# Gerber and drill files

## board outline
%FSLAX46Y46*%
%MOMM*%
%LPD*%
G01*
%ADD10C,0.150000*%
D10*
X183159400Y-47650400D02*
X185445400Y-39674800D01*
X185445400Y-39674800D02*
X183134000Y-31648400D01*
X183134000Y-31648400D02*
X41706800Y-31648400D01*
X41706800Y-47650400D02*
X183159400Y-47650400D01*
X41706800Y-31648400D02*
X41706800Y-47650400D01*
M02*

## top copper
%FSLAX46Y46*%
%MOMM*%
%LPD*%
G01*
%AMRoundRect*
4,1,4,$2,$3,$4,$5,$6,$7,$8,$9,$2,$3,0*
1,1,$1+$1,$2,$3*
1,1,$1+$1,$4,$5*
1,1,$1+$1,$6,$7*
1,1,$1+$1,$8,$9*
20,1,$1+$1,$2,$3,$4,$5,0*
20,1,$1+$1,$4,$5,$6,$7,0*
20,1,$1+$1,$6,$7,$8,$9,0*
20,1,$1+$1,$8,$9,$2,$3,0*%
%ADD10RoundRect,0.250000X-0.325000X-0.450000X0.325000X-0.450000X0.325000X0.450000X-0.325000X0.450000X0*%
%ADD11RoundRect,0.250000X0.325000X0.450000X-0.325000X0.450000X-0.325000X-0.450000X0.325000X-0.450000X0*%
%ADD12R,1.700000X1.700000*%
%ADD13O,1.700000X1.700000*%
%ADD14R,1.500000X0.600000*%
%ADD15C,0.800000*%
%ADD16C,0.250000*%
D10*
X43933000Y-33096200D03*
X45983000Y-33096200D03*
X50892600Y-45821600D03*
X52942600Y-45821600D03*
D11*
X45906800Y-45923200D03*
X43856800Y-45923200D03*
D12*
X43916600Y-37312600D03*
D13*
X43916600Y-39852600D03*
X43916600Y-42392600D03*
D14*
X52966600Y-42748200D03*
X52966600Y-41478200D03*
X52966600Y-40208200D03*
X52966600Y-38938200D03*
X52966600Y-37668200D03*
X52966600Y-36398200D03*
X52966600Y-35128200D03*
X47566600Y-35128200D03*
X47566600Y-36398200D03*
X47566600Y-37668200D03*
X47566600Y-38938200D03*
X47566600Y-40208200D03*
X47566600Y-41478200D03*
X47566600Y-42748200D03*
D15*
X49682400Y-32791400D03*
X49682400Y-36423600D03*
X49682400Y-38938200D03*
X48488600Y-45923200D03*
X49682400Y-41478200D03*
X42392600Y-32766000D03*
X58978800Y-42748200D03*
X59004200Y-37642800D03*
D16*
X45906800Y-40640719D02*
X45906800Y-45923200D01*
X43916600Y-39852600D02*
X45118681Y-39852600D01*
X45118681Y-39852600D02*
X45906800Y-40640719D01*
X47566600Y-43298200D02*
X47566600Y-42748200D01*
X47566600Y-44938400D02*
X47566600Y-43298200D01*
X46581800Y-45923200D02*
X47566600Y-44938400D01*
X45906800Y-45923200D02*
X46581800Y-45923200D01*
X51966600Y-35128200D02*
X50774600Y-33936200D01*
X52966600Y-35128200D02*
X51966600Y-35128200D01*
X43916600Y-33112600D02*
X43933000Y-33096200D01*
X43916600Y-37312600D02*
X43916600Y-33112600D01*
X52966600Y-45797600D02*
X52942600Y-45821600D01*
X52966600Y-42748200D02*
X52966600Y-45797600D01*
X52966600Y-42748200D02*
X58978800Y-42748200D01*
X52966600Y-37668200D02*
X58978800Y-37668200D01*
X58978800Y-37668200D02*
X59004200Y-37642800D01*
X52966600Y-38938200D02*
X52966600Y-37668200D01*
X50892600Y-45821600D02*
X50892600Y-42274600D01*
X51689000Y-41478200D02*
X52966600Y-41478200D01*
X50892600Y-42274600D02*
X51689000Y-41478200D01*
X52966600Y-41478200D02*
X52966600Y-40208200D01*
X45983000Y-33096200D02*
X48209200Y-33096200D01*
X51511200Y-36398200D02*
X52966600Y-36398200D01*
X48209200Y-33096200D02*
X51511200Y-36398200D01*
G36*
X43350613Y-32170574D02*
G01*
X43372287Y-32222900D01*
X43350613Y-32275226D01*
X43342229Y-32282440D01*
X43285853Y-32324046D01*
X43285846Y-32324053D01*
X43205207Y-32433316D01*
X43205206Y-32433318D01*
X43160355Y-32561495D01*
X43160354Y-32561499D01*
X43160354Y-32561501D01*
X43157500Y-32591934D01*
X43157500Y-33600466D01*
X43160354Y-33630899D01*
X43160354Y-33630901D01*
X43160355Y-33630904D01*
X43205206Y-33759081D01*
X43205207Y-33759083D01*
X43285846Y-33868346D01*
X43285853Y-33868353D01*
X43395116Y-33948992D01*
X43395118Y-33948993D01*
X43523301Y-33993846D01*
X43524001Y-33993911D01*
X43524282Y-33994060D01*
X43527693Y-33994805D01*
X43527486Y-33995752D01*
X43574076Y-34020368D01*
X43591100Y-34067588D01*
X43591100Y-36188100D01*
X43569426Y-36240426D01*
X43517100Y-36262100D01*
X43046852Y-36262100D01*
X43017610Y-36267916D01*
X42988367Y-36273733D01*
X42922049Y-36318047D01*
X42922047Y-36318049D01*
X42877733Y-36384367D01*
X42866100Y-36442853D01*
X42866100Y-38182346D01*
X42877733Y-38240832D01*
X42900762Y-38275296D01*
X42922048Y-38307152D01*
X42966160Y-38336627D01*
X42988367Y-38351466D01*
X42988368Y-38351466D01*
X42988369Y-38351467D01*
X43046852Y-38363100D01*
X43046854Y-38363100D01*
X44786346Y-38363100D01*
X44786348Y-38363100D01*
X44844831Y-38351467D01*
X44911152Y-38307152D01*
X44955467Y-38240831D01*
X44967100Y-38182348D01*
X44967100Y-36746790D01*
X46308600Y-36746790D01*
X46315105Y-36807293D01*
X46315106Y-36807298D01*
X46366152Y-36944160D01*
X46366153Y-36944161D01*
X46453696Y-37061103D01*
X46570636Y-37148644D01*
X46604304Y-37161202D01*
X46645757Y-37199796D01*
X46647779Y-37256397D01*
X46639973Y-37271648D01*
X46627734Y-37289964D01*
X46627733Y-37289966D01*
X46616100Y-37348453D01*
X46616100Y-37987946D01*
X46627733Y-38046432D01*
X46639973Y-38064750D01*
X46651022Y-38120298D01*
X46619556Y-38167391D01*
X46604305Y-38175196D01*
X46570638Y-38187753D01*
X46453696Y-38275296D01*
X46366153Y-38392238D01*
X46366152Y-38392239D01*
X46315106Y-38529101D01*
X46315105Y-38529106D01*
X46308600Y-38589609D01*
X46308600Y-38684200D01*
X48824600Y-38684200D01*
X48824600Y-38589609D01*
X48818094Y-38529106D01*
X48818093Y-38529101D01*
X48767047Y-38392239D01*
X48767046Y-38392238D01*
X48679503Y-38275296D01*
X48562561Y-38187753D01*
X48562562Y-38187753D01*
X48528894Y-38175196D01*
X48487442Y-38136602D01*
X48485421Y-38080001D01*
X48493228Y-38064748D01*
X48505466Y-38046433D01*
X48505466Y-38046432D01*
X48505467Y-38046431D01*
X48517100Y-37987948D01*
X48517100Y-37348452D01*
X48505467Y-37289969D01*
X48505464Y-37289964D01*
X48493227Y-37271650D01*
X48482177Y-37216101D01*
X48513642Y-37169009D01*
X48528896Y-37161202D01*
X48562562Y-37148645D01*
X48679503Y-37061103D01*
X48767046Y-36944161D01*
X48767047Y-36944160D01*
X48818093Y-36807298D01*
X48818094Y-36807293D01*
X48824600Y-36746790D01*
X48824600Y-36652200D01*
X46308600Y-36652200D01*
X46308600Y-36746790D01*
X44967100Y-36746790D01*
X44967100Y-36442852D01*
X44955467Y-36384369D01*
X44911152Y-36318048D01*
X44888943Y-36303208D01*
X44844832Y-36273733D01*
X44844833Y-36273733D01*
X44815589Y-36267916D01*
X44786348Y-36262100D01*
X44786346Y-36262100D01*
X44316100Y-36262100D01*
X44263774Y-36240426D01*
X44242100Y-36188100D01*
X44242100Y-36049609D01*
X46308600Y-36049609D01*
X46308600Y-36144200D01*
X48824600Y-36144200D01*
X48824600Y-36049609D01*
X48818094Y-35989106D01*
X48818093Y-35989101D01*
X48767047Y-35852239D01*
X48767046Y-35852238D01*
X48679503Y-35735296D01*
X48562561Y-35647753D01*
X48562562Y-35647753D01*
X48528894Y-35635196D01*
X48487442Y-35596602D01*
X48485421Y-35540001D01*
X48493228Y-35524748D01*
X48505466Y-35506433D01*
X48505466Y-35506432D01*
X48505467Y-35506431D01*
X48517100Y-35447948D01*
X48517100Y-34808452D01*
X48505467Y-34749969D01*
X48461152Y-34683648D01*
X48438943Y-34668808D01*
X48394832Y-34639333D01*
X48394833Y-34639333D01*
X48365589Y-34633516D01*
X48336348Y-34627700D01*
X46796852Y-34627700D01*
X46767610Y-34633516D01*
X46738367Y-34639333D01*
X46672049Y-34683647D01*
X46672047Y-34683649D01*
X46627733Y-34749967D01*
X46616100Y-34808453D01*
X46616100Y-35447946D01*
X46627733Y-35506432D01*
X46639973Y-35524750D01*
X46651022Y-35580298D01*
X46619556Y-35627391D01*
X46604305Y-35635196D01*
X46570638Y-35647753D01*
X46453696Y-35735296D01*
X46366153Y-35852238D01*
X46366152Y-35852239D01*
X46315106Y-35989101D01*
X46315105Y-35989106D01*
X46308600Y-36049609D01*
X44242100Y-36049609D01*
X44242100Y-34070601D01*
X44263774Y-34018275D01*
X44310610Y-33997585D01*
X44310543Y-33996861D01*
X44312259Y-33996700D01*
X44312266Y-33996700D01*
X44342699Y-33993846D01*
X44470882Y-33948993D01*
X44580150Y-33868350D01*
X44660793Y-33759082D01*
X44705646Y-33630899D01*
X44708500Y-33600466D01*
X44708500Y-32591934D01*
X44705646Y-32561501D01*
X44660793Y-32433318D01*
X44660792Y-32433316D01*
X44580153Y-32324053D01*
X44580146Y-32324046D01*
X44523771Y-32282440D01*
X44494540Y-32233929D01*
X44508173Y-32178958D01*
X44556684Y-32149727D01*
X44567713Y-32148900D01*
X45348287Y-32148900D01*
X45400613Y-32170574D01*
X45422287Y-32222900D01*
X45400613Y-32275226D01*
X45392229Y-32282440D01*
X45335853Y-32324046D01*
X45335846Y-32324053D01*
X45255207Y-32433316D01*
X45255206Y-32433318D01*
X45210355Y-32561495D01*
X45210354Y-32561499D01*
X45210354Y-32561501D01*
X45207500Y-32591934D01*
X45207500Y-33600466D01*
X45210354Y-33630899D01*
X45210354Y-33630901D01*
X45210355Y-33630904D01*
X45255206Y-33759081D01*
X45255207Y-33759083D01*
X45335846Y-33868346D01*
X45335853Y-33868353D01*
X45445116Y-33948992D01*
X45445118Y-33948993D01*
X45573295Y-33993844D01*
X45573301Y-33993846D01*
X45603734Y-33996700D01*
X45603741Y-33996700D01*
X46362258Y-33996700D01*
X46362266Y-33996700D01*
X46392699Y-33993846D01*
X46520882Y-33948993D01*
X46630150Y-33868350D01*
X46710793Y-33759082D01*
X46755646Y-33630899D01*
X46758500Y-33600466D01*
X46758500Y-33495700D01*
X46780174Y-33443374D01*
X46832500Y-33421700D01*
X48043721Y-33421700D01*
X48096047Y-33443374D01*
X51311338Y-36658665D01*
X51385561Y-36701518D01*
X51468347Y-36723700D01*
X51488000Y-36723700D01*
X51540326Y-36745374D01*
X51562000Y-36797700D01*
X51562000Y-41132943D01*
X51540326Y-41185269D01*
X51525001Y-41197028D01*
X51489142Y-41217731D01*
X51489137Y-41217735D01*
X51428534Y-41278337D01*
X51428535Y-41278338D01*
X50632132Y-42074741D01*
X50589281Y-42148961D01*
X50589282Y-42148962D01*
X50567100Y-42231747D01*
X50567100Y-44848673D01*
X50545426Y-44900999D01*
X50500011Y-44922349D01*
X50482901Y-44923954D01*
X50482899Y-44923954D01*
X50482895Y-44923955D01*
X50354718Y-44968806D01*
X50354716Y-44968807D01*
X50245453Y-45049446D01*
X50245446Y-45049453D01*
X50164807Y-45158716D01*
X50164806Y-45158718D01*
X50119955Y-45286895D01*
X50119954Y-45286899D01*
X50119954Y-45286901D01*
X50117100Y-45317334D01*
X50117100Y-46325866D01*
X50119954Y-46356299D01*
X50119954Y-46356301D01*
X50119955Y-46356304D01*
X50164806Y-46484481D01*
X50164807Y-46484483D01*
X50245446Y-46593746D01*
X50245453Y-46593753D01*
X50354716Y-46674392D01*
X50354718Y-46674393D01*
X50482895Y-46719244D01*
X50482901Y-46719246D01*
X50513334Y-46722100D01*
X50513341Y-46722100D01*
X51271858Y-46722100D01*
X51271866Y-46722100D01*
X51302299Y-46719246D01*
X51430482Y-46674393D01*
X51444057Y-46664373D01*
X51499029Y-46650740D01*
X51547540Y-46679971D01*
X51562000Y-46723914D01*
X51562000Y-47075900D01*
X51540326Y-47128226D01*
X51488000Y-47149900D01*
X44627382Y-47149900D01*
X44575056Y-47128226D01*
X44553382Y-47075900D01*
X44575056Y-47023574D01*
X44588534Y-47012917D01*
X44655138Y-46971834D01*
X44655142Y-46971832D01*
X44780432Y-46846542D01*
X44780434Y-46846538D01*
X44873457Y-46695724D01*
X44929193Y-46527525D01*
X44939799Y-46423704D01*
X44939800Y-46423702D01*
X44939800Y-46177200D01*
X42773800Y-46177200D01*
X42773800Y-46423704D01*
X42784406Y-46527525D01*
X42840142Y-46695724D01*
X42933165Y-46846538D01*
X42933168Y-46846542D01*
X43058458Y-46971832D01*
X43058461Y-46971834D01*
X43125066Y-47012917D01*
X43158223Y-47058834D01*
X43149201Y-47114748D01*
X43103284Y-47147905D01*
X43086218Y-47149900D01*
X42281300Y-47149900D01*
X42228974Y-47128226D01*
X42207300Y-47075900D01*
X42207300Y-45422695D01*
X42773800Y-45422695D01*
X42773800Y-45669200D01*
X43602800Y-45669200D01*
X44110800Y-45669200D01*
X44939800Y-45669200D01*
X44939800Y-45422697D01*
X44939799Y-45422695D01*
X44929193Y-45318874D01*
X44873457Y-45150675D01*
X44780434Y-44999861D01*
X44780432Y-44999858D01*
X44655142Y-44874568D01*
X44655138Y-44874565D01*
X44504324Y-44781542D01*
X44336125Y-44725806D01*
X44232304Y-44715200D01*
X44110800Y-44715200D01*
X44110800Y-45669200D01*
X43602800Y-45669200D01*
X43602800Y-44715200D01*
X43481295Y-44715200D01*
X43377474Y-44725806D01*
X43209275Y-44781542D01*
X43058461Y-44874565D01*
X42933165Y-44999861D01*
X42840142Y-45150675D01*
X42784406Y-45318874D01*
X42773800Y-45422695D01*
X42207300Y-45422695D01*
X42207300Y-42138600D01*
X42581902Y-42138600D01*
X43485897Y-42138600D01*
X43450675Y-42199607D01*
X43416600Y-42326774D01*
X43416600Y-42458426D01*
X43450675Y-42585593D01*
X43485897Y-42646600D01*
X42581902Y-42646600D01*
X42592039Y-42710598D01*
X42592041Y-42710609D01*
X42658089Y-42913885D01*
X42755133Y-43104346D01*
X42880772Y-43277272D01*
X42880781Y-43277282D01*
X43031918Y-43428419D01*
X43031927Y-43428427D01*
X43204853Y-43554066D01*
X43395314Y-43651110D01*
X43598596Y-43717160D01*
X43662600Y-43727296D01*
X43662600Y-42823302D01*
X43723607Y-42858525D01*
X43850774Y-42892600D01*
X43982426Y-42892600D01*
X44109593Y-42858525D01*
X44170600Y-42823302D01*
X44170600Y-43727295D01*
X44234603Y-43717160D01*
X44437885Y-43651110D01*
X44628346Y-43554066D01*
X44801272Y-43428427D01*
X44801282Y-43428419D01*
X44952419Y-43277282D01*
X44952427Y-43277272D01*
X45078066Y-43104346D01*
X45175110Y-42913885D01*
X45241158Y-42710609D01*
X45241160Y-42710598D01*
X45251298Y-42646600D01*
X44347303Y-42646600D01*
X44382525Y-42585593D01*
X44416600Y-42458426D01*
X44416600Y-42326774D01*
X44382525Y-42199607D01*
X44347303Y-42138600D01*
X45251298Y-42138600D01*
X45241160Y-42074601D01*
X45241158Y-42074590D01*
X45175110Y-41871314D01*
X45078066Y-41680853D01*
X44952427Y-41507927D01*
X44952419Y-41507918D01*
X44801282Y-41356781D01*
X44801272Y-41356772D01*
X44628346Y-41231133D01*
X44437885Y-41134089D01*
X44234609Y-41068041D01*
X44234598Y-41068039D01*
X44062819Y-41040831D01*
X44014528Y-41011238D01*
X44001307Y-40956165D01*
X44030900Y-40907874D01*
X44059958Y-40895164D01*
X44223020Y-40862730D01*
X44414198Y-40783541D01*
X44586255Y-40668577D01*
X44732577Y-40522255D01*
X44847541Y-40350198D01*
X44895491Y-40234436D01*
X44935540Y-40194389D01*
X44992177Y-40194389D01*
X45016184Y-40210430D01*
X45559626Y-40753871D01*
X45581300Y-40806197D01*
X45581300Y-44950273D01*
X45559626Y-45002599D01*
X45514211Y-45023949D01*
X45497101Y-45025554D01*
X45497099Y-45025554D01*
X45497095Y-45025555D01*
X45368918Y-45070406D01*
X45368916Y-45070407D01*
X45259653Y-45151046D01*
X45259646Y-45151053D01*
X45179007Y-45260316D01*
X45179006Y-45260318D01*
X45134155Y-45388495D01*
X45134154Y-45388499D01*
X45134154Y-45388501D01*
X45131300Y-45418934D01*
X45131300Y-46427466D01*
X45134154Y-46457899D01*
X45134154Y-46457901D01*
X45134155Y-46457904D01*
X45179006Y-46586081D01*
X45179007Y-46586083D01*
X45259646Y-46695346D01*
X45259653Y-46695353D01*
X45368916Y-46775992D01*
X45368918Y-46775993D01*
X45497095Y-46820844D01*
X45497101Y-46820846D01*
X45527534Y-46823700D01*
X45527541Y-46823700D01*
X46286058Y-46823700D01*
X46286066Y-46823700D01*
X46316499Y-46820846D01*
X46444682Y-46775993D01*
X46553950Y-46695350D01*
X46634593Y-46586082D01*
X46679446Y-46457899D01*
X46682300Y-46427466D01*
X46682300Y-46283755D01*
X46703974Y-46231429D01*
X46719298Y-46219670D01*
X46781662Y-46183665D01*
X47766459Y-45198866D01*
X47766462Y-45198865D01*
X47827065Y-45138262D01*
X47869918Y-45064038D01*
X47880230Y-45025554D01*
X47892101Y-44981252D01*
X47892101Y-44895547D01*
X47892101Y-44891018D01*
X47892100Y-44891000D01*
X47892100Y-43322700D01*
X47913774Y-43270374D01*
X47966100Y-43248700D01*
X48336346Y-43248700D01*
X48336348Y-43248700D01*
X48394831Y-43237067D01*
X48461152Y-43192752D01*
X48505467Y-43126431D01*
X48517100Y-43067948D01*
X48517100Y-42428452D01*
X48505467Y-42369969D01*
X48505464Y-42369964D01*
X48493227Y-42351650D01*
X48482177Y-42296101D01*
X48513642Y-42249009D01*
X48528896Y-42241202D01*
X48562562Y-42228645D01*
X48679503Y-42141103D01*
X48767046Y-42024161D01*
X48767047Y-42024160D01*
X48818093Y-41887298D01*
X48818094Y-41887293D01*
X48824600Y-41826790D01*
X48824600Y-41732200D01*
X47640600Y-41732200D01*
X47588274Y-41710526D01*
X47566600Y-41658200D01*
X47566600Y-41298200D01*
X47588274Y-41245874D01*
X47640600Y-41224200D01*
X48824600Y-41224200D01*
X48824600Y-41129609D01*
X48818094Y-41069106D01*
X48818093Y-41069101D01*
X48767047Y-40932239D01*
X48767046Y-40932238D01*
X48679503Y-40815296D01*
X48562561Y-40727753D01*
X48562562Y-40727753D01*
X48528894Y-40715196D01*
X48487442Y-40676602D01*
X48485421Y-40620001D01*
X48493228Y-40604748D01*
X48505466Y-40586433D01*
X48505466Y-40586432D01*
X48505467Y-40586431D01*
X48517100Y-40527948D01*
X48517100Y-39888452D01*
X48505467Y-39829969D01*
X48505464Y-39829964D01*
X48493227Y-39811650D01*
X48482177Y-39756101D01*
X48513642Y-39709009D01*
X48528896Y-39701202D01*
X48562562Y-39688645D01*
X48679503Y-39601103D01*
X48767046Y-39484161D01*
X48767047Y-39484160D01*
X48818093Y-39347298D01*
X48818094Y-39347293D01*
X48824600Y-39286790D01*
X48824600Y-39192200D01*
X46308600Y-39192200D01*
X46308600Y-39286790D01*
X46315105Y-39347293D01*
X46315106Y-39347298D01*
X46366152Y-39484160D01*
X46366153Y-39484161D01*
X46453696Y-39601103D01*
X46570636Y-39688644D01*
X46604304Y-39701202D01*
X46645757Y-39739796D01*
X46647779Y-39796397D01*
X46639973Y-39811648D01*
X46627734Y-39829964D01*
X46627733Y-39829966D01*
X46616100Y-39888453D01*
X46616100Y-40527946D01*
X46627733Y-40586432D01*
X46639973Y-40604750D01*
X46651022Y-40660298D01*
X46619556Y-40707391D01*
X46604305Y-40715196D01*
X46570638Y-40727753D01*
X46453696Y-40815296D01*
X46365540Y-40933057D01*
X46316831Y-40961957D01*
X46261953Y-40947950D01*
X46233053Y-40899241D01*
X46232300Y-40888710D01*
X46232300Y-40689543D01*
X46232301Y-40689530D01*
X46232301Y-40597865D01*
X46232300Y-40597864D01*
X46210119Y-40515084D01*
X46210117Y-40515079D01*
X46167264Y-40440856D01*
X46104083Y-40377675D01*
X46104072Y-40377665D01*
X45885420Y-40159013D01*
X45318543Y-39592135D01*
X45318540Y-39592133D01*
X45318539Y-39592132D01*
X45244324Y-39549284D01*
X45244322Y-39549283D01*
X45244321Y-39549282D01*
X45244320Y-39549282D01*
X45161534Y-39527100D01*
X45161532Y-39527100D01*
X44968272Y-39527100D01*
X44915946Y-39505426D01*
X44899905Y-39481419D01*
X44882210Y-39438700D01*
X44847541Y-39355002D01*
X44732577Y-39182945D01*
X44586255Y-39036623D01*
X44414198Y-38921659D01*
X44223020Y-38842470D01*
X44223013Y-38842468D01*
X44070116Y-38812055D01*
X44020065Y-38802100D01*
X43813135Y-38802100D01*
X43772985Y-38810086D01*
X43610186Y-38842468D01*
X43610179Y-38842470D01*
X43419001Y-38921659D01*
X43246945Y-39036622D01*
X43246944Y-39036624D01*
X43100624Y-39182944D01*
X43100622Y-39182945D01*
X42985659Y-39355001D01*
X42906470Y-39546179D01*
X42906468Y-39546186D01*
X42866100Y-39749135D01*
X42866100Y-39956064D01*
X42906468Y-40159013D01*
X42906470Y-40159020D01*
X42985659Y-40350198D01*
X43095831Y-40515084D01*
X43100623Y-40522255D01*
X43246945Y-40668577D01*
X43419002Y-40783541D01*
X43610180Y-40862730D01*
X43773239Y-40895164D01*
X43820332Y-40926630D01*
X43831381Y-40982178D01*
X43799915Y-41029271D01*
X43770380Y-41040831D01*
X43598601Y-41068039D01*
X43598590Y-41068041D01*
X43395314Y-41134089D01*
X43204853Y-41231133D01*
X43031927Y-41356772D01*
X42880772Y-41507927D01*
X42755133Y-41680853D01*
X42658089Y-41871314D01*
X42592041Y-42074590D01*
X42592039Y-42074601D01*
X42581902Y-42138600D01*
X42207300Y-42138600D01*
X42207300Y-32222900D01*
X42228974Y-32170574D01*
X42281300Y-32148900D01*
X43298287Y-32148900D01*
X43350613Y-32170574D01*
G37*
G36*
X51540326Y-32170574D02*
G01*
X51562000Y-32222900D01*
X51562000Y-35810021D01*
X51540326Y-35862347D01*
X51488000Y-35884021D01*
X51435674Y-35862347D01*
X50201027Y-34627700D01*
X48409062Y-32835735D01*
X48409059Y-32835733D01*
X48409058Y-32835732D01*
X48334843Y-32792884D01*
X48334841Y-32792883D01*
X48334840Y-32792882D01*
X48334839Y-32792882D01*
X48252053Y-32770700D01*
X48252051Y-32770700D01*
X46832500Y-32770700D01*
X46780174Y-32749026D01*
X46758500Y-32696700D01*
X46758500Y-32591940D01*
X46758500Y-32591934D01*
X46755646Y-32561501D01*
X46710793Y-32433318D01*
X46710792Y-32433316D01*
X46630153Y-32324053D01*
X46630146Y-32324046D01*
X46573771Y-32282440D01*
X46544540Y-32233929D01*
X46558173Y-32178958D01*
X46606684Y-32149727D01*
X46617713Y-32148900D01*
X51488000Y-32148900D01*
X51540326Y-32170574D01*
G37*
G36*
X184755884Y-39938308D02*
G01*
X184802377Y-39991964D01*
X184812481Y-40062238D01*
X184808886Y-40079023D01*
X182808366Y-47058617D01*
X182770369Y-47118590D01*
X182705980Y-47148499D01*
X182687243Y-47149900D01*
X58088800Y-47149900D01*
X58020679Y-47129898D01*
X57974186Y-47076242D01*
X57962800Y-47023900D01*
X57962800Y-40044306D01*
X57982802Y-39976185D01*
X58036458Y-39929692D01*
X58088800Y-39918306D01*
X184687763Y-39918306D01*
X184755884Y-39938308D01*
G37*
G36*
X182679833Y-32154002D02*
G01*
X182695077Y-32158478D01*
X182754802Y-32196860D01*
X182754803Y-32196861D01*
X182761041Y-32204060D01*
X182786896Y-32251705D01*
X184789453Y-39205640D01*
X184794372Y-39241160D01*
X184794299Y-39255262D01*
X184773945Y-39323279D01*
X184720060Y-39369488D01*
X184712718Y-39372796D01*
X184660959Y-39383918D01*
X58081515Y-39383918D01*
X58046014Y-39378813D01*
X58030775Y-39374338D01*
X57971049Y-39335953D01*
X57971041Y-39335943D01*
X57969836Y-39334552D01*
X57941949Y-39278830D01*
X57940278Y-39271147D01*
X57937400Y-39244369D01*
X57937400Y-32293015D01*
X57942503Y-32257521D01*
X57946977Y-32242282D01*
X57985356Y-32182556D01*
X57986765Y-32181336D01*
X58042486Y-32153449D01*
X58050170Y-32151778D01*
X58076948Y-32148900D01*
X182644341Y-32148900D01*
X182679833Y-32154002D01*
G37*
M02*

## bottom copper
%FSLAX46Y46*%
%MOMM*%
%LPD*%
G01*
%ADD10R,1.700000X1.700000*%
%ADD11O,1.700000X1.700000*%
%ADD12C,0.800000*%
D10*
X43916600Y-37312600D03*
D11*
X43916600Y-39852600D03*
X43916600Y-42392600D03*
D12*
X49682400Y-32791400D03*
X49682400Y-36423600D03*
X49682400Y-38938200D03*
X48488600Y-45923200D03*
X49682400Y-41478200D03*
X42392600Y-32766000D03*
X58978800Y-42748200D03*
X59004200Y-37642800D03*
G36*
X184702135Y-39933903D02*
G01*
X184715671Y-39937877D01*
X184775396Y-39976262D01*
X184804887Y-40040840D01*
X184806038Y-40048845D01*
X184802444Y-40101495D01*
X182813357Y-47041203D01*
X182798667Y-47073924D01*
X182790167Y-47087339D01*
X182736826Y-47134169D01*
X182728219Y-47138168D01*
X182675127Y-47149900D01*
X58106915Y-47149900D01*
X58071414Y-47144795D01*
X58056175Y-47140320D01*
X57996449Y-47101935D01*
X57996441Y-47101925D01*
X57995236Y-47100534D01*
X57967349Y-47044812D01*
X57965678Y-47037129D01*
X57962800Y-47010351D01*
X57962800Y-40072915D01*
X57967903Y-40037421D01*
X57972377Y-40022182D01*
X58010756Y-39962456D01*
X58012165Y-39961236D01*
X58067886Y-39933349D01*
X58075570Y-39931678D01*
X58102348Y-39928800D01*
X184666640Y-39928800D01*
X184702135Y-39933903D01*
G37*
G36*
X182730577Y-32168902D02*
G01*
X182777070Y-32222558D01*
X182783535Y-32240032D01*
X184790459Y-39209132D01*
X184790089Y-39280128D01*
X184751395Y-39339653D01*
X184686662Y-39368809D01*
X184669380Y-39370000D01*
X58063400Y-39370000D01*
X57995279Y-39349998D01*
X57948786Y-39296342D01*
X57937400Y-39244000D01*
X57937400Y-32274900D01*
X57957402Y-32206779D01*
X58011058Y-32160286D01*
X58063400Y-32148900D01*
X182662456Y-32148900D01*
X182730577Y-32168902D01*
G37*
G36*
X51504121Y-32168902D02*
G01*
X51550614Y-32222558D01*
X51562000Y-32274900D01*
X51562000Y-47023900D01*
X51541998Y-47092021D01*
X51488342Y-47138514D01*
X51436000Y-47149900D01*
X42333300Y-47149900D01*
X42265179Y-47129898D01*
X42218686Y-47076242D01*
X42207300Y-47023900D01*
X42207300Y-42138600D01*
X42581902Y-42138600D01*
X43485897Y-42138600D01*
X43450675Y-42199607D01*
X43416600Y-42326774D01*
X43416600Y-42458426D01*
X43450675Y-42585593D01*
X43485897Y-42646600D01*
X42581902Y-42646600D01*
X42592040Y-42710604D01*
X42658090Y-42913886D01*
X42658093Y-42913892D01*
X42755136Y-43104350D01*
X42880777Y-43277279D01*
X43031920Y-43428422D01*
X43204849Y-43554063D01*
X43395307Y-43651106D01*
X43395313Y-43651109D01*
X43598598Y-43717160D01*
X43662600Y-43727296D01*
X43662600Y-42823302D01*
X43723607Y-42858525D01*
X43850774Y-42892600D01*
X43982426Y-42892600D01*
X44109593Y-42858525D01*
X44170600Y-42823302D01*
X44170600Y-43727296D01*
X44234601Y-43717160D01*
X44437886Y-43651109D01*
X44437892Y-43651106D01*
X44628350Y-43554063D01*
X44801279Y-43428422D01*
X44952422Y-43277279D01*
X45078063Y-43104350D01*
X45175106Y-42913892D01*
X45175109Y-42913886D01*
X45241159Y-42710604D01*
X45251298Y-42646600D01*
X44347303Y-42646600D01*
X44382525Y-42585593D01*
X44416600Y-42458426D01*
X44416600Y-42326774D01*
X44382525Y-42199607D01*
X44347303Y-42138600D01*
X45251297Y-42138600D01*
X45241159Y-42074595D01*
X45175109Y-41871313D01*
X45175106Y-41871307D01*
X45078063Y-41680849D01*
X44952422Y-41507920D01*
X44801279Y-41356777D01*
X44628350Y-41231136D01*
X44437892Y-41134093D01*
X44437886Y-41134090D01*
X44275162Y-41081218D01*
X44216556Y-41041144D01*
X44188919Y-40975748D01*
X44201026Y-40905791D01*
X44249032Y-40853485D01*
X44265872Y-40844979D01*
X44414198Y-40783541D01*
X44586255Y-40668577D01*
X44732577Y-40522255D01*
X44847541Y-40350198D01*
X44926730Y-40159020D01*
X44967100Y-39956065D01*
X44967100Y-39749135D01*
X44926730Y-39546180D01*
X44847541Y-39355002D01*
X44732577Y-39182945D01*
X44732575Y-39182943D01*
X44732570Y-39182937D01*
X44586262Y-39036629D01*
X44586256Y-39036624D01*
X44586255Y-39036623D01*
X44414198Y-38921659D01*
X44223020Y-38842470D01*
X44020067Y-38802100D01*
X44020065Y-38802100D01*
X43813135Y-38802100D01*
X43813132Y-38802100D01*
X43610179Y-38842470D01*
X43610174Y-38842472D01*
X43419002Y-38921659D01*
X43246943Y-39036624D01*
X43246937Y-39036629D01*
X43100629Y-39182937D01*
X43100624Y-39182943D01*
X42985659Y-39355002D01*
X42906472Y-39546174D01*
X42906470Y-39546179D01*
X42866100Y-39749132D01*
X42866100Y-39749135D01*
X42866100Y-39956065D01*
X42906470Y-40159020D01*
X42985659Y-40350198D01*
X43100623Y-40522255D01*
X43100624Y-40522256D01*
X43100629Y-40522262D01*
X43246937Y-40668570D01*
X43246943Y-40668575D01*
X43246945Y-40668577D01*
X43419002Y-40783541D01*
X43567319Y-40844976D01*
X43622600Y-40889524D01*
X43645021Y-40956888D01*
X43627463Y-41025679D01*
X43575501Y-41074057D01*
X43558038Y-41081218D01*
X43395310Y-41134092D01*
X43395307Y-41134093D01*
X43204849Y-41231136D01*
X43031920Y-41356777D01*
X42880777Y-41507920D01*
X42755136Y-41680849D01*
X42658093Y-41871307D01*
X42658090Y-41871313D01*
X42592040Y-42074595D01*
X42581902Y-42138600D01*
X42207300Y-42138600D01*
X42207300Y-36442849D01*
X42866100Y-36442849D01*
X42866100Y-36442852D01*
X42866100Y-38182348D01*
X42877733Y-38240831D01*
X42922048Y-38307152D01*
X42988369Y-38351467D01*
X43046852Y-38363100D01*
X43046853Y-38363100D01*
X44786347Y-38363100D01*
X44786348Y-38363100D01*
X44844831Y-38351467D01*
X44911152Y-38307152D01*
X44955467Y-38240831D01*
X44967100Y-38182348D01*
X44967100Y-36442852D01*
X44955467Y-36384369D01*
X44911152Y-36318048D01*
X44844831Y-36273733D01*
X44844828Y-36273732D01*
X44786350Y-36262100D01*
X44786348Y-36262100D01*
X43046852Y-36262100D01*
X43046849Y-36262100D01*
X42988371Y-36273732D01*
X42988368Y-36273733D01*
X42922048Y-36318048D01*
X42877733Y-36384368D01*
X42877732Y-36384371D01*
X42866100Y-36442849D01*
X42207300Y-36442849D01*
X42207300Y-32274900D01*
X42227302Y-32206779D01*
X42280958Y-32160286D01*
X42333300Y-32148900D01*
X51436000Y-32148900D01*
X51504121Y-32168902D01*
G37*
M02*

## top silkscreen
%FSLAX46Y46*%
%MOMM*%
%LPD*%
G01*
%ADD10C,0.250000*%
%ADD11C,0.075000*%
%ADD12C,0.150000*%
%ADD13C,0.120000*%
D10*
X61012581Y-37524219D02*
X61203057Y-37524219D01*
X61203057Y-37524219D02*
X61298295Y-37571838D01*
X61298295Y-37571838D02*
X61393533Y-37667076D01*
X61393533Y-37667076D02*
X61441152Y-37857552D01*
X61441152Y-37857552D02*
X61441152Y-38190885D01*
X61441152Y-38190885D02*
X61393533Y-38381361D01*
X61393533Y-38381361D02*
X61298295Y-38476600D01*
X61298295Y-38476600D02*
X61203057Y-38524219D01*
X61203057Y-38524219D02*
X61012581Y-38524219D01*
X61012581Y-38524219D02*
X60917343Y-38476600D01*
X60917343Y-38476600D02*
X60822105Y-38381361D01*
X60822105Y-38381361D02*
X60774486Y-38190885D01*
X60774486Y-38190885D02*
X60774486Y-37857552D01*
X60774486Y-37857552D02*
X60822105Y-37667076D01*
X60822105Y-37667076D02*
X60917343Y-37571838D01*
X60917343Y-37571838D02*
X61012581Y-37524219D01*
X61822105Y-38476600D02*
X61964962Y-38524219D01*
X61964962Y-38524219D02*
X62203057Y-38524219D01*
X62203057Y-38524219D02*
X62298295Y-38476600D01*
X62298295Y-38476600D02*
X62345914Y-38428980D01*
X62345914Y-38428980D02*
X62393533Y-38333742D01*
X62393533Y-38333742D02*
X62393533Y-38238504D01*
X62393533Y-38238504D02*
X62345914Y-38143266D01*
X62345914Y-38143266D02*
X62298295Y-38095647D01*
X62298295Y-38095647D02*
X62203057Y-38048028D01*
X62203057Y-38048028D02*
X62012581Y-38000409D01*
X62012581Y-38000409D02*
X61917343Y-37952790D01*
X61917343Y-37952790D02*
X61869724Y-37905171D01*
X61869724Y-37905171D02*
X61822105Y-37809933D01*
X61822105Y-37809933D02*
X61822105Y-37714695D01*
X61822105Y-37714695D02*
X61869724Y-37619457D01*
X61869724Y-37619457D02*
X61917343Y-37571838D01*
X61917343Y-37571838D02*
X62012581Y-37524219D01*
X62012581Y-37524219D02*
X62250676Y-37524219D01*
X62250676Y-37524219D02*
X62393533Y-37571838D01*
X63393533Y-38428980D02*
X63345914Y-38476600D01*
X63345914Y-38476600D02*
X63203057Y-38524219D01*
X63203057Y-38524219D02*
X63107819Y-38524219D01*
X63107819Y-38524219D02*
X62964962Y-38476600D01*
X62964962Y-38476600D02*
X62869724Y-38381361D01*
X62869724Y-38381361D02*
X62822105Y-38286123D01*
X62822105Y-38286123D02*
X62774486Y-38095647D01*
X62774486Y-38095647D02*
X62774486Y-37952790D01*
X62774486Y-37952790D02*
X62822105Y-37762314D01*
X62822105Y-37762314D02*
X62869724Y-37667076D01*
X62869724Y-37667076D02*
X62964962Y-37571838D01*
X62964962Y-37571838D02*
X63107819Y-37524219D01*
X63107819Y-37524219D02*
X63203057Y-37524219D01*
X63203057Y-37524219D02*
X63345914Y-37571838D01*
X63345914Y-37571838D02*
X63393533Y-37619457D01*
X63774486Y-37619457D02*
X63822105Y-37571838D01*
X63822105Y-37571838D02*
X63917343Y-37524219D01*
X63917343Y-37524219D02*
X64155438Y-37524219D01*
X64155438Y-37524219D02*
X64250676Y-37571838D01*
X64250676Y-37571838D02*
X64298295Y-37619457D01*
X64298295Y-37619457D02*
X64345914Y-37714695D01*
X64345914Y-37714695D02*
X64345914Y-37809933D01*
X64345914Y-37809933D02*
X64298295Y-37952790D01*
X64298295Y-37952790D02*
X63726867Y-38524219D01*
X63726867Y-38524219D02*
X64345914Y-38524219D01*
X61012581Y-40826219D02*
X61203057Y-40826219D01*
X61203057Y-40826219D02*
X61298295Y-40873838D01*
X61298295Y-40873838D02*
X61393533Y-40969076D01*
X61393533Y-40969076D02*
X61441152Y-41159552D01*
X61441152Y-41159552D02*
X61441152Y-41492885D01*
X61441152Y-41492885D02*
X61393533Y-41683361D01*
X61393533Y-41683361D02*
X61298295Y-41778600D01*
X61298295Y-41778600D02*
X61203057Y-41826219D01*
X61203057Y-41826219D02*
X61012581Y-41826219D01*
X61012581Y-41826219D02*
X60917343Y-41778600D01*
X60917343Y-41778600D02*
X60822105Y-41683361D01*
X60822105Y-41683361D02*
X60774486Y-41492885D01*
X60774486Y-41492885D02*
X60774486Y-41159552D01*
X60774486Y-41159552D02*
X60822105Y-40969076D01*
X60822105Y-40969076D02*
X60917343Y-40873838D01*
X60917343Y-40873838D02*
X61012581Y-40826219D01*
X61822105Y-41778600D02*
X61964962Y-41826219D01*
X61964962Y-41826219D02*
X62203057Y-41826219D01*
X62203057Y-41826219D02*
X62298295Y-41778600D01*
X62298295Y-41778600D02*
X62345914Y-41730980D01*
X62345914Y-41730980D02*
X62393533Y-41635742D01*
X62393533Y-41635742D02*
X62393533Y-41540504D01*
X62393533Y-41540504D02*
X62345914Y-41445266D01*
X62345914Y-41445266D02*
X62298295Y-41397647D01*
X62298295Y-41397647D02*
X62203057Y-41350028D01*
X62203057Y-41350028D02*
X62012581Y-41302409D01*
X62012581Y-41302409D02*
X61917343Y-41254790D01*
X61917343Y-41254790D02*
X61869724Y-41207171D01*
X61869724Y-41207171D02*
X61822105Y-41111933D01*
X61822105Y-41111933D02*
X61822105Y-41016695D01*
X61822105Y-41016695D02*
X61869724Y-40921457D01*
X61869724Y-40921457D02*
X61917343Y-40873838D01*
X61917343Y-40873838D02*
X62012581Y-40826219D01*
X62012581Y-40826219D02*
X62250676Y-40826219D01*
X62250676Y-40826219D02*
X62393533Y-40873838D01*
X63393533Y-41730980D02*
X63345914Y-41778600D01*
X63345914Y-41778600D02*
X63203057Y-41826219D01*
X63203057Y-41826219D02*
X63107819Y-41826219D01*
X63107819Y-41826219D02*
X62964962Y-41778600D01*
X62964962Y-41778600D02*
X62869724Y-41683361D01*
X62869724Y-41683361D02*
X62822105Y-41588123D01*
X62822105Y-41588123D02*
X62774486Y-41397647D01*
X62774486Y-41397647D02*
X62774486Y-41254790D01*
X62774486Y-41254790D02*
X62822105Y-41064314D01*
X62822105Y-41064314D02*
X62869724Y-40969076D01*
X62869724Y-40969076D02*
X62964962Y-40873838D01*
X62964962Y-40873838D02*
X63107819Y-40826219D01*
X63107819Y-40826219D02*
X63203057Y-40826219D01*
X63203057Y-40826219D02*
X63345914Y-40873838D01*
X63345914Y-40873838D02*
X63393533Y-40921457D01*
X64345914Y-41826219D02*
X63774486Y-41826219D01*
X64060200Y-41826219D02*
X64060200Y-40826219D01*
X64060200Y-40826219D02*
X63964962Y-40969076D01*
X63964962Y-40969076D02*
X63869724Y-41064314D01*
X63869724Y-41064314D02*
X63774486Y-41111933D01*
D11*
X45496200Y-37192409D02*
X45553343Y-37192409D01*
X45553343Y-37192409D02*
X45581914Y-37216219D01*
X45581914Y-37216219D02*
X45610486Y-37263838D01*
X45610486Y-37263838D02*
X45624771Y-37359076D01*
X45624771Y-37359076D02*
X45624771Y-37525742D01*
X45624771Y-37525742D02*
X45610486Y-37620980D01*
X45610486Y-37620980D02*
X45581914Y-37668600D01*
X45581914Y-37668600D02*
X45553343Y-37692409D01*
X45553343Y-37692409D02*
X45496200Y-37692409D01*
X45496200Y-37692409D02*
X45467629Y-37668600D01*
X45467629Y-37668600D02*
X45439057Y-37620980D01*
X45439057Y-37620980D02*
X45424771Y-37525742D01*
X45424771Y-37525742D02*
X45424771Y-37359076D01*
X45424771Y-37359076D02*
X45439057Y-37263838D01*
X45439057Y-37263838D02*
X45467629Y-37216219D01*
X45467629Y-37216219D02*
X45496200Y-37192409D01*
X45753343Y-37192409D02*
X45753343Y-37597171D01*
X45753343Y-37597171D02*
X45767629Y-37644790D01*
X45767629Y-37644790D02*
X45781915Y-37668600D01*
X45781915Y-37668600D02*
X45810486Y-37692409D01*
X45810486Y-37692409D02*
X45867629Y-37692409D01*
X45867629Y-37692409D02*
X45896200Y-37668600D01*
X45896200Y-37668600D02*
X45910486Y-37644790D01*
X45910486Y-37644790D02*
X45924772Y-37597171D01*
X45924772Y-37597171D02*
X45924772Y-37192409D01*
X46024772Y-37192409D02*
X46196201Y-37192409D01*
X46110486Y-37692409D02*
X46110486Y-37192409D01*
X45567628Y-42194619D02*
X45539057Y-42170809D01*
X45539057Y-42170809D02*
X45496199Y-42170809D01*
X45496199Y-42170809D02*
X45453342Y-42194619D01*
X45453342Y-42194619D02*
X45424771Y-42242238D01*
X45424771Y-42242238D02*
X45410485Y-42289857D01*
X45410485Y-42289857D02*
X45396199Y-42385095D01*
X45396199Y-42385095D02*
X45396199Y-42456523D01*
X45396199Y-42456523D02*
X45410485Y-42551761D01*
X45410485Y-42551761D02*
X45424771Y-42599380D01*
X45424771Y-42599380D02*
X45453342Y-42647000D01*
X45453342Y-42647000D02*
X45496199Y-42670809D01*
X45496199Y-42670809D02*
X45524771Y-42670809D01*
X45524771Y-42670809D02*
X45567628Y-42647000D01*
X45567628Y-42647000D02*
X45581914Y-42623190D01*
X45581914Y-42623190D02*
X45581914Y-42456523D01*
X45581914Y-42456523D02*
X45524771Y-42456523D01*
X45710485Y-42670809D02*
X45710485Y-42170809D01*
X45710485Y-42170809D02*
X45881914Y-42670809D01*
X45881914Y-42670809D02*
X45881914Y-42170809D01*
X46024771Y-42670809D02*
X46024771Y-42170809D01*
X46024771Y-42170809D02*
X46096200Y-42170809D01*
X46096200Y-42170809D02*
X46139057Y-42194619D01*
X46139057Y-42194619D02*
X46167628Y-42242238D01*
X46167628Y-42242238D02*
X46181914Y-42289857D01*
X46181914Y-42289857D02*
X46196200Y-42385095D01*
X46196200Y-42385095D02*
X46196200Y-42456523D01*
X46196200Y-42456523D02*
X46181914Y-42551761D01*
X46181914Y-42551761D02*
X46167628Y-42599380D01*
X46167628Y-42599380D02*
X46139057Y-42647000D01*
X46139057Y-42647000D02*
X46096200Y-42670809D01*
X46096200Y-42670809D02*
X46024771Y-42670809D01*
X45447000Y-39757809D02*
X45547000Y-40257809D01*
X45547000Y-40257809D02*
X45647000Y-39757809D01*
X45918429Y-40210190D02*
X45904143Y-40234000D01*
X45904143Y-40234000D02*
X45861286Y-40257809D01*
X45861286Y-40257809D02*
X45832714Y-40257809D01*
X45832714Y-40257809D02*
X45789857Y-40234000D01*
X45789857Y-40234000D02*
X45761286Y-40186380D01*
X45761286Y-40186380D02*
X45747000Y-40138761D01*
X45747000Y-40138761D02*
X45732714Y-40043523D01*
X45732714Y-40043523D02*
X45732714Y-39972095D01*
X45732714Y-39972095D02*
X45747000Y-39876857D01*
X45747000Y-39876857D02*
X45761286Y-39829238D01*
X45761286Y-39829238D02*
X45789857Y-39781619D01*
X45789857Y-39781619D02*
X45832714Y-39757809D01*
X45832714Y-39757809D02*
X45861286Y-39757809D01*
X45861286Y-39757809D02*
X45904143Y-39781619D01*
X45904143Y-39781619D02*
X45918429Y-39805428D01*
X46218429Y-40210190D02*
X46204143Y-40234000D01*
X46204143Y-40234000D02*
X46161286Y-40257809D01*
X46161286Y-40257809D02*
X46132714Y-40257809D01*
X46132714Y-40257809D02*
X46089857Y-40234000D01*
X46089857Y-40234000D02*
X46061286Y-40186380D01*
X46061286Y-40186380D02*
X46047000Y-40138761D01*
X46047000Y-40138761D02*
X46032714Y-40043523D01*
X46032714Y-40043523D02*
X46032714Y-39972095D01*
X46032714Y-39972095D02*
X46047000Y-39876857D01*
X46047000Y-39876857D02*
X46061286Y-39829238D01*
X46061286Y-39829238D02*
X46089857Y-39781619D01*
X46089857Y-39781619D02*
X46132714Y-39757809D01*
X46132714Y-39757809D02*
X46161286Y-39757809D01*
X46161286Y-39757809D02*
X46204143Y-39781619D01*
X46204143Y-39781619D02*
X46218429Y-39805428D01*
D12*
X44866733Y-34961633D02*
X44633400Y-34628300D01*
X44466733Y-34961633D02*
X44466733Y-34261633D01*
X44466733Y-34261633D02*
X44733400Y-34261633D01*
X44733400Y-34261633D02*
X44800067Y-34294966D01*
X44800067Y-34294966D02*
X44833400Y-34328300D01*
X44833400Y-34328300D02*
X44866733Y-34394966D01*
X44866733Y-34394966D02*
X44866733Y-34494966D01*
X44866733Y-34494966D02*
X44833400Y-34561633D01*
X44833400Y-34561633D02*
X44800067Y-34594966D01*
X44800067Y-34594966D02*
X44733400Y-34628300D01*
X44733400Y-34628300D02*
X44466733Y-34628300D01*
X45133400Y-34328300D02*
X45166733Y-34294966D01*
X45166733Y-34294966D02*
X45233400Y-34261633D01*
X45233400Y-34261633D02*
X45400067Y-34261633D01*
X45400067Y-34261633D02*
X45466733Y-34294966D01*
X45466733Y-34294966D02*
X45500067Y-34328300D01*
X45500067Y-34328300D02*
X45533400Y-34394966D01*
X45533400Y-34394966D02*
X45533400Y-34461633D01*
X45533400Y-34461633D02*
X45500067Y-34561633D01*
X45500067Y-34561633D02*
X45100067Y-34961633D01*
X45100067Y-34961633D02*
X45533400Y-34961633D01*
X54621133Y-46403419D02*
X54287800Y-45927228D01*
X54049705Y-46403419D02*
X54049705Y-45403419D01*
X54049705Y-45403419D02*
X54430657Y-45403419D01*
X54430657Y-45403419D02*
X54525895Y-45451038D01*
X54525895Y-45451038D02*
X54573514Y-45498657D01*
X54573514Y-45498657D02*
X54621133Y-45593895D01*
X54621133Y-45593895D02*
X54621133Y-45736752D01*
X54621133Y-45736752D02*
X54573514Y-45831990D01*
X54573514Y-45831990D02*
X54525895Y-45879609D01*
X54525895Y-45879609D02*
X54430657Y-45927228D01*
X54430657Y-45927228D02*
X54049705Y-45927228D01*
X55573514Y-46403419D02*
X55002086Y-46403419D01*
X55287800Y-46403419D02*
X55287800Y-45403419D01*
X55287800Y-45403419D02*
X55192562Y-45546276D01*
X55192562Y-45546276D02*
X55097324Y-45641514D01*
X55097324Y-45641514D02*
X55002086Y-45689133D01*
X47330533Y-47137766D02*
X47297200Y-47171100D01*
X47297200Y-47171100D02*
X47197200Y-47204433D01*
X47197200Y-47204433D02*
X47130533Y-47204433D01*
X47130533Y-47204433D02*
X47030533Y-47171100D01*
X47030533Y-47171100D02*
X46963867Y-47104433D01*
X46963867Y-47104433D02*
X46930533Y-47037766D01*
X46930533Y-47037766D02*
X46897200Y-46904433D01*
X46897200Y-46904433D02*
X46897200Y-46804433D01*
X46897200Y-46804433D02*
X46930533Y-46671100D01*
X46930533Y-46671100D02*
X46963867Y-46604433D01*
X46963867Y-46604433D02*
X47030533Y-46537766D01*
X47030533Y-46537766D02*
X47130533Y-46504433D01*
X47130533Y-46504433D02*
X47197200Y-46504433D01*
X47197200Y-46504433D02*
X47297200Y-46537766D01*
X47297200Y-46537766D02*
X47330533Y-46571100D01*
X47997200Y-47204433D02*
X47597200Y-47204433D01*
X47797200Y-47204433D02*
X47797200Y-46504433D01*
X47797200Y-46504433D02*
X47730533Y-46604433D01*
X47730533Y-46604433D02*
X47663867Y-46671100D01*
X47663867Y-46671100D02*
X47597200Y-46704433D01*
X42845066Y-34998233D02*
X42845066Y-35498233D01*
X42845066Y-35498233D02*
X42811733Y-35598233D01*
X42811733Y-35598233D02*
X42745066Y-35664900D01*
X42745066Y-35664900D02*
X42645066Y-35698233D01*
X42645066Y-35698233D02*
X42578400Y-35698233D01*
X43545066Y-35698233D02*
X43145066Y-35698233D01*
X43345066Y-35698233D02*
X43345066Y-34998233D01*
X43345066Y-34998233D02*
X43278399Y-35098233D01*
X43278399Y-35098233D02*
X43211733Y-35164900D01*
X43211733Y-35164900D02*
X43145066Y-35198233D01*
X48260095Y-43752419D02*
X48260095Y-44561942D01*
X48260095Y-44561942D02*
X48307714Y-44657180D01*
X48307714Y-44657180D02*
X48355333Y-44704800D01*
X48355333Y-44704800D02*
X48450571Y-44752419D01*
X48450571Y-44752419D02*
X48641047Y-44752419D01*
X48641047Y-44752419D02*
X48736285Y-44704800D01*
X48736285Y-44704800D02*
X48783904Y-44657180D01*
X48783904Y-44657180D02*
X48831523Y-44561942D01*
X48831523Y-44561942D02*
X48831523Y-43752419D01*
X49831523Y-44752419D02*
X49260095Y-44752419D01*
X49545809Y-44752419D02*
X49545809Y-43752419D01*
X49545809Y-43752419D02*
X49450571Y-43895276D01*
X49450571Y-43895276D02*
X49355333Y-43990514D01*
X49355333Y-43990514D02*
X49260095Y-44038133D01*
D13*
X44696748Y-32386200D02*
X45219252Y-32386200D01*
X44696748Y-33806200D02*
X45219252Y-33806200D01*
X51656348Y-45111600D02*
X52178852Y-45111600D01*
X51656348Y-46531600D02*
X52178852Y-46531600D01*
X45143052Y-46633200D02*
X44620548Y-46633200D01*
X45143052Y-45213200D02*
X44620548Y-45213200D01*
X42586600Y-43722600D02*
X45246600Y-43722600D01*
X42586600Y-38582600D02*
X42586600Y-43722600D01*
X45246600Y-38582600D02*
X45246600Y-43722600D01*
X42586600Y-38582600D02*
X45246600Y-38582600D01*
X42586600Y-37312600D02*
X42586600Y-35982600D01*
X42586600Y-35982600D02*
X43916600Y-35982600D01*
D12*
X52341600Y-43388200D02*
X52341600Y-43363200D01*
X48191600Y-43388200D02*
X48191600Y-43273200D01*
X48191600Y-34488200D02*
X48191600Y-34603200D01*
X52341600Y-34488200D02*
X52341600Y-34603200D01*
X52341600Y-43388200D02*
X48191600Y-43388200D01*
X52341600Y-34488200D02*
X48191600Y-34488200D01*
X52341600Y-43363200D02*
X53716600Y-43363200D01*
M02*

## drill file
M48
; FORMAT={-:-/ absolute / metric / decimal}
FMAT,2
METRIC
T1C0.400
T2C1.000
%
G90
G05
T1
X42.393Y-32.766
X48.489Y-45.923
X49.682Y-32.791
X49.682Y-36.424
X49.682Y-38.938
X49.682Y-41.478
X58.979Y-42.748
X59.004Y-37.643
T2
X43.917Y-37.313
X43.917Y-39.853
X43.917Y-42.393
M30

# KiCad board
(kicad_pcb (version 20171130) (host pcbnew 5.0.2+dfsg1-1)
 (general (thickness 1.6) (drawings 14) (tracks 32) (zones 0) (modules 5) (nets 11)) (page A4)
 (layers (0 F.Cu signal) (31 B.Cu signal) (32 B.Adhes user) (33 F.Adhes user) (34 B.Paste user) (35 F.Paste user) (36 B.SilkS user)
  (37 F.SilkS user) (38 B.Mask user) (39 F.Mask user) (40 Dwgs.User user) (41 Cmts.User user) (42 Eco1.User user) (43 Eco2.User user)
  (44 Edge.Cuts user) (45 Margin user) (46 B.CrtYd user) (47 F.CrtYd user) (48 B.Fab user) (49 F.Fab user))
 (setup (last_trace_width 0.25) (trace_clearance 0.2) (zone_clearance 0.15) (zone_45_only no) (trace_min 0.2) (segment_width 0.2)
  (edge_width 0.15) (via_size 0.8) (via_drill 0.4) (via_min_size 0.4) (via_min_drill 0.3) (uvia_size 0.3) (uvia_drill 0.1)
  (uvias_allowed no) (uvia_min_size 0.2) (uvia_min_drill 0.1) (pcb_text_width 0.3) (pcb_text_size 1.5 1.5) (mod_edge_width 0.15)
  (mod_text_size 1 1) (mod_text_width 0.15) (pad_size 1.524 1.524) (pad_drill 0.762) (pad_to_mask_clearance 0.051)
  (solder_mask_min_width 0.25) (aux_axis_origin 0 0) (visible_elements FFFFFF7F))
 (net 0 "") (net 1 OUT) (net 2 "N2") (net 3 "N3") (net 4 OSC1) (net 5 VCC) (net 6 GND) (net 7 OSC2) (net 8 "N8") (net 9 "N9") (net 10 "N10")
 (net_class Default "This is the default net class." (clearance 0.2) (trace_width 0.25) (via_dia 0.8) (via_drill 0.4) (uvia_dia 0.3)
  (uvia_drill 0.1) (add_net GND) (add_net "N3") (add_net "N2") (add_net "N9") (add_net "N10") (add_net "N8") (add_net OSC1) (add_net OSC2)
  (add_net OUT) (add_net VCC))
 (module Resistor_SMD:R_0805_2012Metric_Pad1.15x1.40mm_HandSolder (layer F.Cu) (at 44.958 33.0962)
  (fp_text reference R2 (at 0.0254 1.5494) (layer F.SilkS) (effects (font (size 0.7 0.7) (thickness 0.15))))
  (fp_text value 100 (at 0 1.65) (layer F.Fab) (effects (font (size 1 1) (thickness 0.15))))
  (fp_line (start -0.261252 -0.71) (end 0.261252 -0.71) (layer F.SilkS) (width 0.12))
  (fp_line (start -0.261252 0.71) (end 0.261252 0.71) (layer F.SilkS) (width 0.12))
  (pad 1 smd roundrect (at -1.025 0) (size 1.15 1.4) (layers F.Cu F.Paste F.Mask) (roundrect_rratio 0.217391) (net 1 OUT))
  (pad 2 smd roundrect (at 1.025 0) (size 1.15 1.4) (layers F.Cu F.Paste F.Mask) (roundrect_rratio 0.217391) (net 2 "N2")))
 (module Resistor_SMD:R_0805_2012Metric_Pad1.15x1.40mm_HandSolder (layer F.Cu) (at 51.9176 45.8216)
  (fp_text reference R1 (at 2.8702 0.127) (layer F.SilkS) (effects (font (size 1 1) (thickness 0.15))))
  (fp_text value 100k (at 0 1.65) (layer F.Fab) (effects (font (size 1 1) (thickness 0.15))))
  (fp_line (start -0.261252 -0.71) (end 0.261252 -0.71) (layer F.SilkS) (width 0.12))
  (fp_line (start -0.261252 0.71) (end 0.261252 0.71) (layer F.SilkS) (width 0.12))
  (pad 1 smd roundrect (at -1.025 0) (size 1.15 1.4) (layers F.Cu F.Paste F.Mask) (roundrect_rratio 0.217391) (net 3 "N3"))
  (pad 2 smd roundrect (at 1.025 0) (size 1.15 1.4) (layers F.Cu F.Paste F.Mask) (roundrect_rratio 0.217391) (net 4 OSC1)))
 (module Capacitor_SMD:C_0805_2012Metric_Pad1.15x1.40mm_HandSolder (layer F.Cu) (at 44.8818 45.9232 180)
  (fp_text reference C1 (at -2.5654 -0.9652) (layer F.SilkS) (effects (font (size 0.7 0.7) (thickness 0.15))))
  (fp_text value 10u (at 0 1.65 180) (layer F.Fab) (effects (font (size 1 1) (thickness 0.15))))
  (fp_line (start -0.261252 -0.71) (end 0.261252 -0.71) (layer F.SilkS) (width 0.12))
  (fp_line (start -0.261252 0.71) (end 0.261252 0.71) (layer F.SilkS) (width 0.12))
  (pad 1 smd roundrect (at -1.025 0 180) (size 1.15 1.4) (layers F.Cu F.Paste F.Mask) (roundrect_rratio 0.217391) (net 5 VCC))
  (pad 2 smd roundrect (at 1.025 0 180) (size 1.15 1.4) (layers F.Cu F.Paste F.Mask) (roundrect_rratio 0.217391) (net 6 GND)))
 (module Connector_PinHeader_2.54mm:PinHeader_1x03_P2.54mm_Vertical (layer F.Cu) (at 43.9166 37.3126)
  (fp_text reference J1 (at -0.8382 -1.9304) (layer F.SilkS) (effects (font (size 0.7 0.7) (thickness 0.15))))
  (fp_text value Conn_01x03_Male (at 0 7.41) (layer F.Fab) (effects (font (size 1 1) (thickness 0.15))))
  (fp_line (start -1.33 6.41) (end 1.33 6.41) (layer F.SilkS) (width 0.12))
  (fp_line (start -1.33 1.27) (end -1.33 6.41) (layer F.SilkS) (width 0.12))
  (fp_line (start 1.33 1.27) (end 1.33 6.41) (layer F.SilkS) (width 0.12))
  (fp_line (start -1.33 1.27) (end 1.33 1.27) (layer F.SilkS) (width 0.12))
  (fp_line (start -1.33 0) (end -1.33 -1.33) (layer F.SilkS) (width 0.12))
  (fp_line (start -1.33 -1.33) (end 0 -1.33) (layer F.SilkS) (width 0.12))
  (pad 1 thru_hole rect (at 0 0) (size 1.7 1.7) (drill 1) (layers *.Cu *.Mask) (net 1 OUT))
  (pad 2 thru_hole oval (at 0 2.54) (size 1.7 1.7) (drill 1) (layers *.Cu *.Mask) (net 5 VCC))
  (pad 3 thru_hole oval (at 0 5.08) (size 1.7 1.7) (drill 1) (layers *.Cu *.Mask) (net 6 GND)))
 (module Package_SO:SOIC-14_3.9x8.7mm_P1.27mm (layer F.Cu) (at 50.2666 38.9382 180)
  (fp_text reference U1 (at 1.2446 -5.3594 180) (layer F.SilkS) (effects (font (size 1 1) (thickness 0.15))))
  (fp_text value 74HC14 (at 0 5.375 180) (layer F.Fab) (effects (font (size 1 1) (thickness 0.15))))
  (fp_line (start -2.075 -4.45) (end -2.075 -4.425) (layer F.SilkS) (width 0.15))
  (fp_line (start 2.075 -4.45) (end 2.075 -4.335) (layer F.SilkS) (width 0.15))
  (fp_line (start 2.075 4.45) (end 2.075 4.335) (layer F.SilkS) (width 0.15))
  (fp_line (start -2.075 4.45) (end -2.075 4.335) (layer F.SilkS) (width 0.15))
  (fp_line (start -2.075 -4.45) (end 2.075 -4.45) (layer F.SilkS) (width 0.15))
  (fp_line (start -2.075 4.45) (end 2.075 4.45) (layer F.SilkS) (width 0.15))
  (fp_line (start -2.075 -4.425) (end -3.45 -4.425) (layer F.SilkS) (width 0.15))
  (pad 1 smd rect (at -2.7 -3.81 180) (size 1.5 0.6) (layers F.Cu F.Paste F.Mask) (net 4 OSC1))
  (pad 2 smd rect (at -2.7 -2.54 180) (size 1.5 0.6) (layers F.Cu F.Paste F.Mask) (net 3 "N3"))
  (pad 3 smd rect (at -2.7 -1.27 180) (size 1.5 0.6) (layers F.Cu F.Paste F.Mask) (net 3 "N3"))
  (pad 4 smd rect (at -2.7 0 180) (size 1.5 0.6) (layers F.Cu F.Paste F.Mask) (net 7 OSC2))
  (pad 5 smd rect (at -2.7 1.27 180) (size 1.5 0.6) (layers F.Cu F.Paste F.Mask) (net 7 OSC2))
  (pad 6 smd rect (at -2.7 2.54 180) (size 1.5 0.6) (layers F.Cu F.Paste F.Mask) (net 2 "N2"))
  (pad 7 smd rect (at -2.7 3.81 180) (size 1.5 0.6) (layers F.Cu F.Paste F.Mask) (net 6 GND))
  (pad 8 smd rect (at 2.7 3.81 180) (size 1.5 0.6) (layers F.Cu F.Paste F.Mask) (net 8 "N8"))
  (pad 9 smd rect (at 2.7 2.54 180) (size 1.5 0.6) (layers F.Cu F.Paste F.Mask) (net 6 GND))
  (pad 10 smd rect (at 2.7 1.27 180) (size 1.5 0.6) (layers F.Cu F.Paste F.Mask) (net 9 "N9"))
  (pad 11 smd rect (at 2.7 0 180) (size 1.5 0.6) (layers F.Cu F.Paste F.Mask) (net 6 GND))
  (pad 12 smd rect (at 2.7 -1.27 180) (size 1.5 0.6) (layers F.Cu F.Paste F.Mask) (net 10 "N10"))
  (pad 13 smd rect (at 2.7 -2.54 180) (size 1.5 0.6) (layers F.Cu F.Paste F.Mask) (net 6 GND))
  (pad 14 smd rect (at 2.7 -3.81 180) (size 1.5 0.6) (layers F.Cu F.Paste F.Mask) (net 5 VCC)))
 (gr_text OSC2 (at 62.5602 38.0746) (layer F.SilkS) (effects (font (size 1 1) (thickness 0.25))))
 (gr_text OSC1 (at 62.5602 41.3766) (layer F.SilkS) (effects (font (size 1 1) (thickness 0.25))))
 (gr_line (start 183.1594 47.6504) (end 185.4454 39.6748) (layer Edge.Cuts) (width 0.15))
 (gr_line (start 185.4454 39.6748) (end 183.134 31.6484) (layer Edge.Cuts) (width 0.15))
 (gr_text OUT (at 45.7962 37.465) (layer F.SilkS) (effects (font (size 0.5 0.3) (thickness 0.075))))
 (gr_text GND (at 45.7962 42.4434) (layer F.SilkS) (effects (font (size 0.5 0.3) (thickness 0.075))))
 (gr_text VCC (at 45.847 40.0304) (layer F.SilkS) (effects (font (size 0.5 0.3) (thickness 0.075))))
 (gr_line (start 183.134 31.6484) (end 41.7068 31.6484) (layer Edge.Cuts) (width 0.15))
 (gr_line (start 41.7068 47.6504) (end 183.1594 47.6504) (layer Edge.Cuts) (width 0.15))
 (gr_line (start 41.7068 31.6484) (end 41.7068 47.6504) (layer Edge.Cuts) (width 0.15))
 (segment (start 45.9068 40.640719) (end 45.9068 45.9232) (width 0.25) (layer F.Cu) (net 5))
 (segment (start 43.9166 39.8526) (end 45.118681 39.8526) (width 0.25) (layer F.Cu) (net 5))
 (segment (start 45.118681 39.8526) (end 45.9068 40.640719) (width 0.25) (layer F.Cu) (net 5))
 (segment (start 47.5666 43.2982) (end 47.5666 42.7482) (width 0.25) (layer F.Cu) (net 5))
 (segment (start 47.5666 44.9384) (end 47.5666 43.2982) (width 0.25) (layer F.Cu) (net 5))
 (segment (start 46.5818 45.9232) (end 47.5666 44.9384) (width 0.25) (layer F.Cu) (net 5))
 (segment (start 45.9068 45.9232) (end 46.5818 45.9232) (width 0.25) (layer F.Cu) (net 5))
 (segment (start 51.9666 35.1282) (end 50.7746 33.9362) (width 0.25) (layer F.Cu) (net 6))
 (segment (start 52.9666 35.1282) (end 51.9666 35.1282) (width 0.25) (layer F.Cu) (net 6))
 (via (at 49.6824 32.7914) (size 0.8) (drill 0.4) (layers F.Cu B.Cu) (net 6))
 (via (at 49.6824 36.4236) (size 0.8) (drill 0.4) (layers F.Cu B.Cu) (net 6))
 (via (at 49.6824 38.9382) (size 0.8) (drill 0.4) (layers F.Cu B.Cu) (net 6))
 (via (at 48.4886 45.9232) (size 0.8) (drill 0.4) (layers F.Cu B.Cu) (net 6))
 (via (at 49.6824 41.4782) (size 0.8) (drill 0.4) (layers F.Cu B.Cu) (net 6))
 (via (at 42.3926 32.766) (size 0.8) (drill 0.4) (layers F.Cu B.Cu) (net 6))
 (segment (start 43.9166 33.1126) (end 43.933 33.0962) (width 0.25) (layer F.Cu) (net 1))
 (segment (start 43.9166 37.3126) (end 43.9166 33.1126) (width 0.25) (layer F.Cu) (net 1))
 (segment (start 52.9666 45.7976) (end 52.9426 45.8216) (width 0.25) (layer F.Cu) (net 4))
 (segment (start 52.9666 42.7482) (end 52.9666 45.7976) (width 0.25) (layer F.Cu) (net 4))
 (via (at 58.9788 42.7482) (size 0.8) (drill 0.4) (layers F.Cu B.Cu) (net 4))
 (segment (start 52.9666 42.7482) (end 58.9788 42.7482) (width 0.25) (layer F.Cu) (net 4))
 (via (at 59.0042 37.6428) (size 0.8) (drill 0.4) (layers F.Cu B.Cu) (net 7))
 (segment (start 52.9666 37.6682) (end 58.9788 37.6682) (width 0.25) (layer F.Cu) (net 7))
 (segment (start 58.9788 37.6682) (end 59.0042 37.6428) (width 0.25) (layer F.Cu) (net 7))
 (segment (start 52.9666 38.9382) (end 52.9666 37.6682) (width 0.25) (layer F.Cu) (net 7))
 (segment (start 50.8926 45.8216) (end 50.8926 42.2746) (width 0.25) (layer F.Cu) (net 3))
 (segment (start 51.689 41.4782) (end 52.9666 41.4782) (width 0.25) (layer F.Cu) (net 3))
 (segment (start 50.8926 42.2746) (end 51.689 41.4782) (width 0.25) (layer F.Cu) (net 3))
 (segment (start 52.9666 41.4782) (end 52.9666 40.2082) (width 0.25) (layer F.Cu) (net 3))
 (segment (start 45.983 33.0962) (end 48.2092 33.0962) (width 0.25) (layer F.Cu) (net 2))
 (segment (start 51.5112 36.3982) (end 52.9666 36.3982) (width 0.25) (layer F.Cu) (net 2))
 (segment (start 48.2092 33.0962) (end 51.5112 36.3982) (width 0.25) (layer F.Cu) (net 2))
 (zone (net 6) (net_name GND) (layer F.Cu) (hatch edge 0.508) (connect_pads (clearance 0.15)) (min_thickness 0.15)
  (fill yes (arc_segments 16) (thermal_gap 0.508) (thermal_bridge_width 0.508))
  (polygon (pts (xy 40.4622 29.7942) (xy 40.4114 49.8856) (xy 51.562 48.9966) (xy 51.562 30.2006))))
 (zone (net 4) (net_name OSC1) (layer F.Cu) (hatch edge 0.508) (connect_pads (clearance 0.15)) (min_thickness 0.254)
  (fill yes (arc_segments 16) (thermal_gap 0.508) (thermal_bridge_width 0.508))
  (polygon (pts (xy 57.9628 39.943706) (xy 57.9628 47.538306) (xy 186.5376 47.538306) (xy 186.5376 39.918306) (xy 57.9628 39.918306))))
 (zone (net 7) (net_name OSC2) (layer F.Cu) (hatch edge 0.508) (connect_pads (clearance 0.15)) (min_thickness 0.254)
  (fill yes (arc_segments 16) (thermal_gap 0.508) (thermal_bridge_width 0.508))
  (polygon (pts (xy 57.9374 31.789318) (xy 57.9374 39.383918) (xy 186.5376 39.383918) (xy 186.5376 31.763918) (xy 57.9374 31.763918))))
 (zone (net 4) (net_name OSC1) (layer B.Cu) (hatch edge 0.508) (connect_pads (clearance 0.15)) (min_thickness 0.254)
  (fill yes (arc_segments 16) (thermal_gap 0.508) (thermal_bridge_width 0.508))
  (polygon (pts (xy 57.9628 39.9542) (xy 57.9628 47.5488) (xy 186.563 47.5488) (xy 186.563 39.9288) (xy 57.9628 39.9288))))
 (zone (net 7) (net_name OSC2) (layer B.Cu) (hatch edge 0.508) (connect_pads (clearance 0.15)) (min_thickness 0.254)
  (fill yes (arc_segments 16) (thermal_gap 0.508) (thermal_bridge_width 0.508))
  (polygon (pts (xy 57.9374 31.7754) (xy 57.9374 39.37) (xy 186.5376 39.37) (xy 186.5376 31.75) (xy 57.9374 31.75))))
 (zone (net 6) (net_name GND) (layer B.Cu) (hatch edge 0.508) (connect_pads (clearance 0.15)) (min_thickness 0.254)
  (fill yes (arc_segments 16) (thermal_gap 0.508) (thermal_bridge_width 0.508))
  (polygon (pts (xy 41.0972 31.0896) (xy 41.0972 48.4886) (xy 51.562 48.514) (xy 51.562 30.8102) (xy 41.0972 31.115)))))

